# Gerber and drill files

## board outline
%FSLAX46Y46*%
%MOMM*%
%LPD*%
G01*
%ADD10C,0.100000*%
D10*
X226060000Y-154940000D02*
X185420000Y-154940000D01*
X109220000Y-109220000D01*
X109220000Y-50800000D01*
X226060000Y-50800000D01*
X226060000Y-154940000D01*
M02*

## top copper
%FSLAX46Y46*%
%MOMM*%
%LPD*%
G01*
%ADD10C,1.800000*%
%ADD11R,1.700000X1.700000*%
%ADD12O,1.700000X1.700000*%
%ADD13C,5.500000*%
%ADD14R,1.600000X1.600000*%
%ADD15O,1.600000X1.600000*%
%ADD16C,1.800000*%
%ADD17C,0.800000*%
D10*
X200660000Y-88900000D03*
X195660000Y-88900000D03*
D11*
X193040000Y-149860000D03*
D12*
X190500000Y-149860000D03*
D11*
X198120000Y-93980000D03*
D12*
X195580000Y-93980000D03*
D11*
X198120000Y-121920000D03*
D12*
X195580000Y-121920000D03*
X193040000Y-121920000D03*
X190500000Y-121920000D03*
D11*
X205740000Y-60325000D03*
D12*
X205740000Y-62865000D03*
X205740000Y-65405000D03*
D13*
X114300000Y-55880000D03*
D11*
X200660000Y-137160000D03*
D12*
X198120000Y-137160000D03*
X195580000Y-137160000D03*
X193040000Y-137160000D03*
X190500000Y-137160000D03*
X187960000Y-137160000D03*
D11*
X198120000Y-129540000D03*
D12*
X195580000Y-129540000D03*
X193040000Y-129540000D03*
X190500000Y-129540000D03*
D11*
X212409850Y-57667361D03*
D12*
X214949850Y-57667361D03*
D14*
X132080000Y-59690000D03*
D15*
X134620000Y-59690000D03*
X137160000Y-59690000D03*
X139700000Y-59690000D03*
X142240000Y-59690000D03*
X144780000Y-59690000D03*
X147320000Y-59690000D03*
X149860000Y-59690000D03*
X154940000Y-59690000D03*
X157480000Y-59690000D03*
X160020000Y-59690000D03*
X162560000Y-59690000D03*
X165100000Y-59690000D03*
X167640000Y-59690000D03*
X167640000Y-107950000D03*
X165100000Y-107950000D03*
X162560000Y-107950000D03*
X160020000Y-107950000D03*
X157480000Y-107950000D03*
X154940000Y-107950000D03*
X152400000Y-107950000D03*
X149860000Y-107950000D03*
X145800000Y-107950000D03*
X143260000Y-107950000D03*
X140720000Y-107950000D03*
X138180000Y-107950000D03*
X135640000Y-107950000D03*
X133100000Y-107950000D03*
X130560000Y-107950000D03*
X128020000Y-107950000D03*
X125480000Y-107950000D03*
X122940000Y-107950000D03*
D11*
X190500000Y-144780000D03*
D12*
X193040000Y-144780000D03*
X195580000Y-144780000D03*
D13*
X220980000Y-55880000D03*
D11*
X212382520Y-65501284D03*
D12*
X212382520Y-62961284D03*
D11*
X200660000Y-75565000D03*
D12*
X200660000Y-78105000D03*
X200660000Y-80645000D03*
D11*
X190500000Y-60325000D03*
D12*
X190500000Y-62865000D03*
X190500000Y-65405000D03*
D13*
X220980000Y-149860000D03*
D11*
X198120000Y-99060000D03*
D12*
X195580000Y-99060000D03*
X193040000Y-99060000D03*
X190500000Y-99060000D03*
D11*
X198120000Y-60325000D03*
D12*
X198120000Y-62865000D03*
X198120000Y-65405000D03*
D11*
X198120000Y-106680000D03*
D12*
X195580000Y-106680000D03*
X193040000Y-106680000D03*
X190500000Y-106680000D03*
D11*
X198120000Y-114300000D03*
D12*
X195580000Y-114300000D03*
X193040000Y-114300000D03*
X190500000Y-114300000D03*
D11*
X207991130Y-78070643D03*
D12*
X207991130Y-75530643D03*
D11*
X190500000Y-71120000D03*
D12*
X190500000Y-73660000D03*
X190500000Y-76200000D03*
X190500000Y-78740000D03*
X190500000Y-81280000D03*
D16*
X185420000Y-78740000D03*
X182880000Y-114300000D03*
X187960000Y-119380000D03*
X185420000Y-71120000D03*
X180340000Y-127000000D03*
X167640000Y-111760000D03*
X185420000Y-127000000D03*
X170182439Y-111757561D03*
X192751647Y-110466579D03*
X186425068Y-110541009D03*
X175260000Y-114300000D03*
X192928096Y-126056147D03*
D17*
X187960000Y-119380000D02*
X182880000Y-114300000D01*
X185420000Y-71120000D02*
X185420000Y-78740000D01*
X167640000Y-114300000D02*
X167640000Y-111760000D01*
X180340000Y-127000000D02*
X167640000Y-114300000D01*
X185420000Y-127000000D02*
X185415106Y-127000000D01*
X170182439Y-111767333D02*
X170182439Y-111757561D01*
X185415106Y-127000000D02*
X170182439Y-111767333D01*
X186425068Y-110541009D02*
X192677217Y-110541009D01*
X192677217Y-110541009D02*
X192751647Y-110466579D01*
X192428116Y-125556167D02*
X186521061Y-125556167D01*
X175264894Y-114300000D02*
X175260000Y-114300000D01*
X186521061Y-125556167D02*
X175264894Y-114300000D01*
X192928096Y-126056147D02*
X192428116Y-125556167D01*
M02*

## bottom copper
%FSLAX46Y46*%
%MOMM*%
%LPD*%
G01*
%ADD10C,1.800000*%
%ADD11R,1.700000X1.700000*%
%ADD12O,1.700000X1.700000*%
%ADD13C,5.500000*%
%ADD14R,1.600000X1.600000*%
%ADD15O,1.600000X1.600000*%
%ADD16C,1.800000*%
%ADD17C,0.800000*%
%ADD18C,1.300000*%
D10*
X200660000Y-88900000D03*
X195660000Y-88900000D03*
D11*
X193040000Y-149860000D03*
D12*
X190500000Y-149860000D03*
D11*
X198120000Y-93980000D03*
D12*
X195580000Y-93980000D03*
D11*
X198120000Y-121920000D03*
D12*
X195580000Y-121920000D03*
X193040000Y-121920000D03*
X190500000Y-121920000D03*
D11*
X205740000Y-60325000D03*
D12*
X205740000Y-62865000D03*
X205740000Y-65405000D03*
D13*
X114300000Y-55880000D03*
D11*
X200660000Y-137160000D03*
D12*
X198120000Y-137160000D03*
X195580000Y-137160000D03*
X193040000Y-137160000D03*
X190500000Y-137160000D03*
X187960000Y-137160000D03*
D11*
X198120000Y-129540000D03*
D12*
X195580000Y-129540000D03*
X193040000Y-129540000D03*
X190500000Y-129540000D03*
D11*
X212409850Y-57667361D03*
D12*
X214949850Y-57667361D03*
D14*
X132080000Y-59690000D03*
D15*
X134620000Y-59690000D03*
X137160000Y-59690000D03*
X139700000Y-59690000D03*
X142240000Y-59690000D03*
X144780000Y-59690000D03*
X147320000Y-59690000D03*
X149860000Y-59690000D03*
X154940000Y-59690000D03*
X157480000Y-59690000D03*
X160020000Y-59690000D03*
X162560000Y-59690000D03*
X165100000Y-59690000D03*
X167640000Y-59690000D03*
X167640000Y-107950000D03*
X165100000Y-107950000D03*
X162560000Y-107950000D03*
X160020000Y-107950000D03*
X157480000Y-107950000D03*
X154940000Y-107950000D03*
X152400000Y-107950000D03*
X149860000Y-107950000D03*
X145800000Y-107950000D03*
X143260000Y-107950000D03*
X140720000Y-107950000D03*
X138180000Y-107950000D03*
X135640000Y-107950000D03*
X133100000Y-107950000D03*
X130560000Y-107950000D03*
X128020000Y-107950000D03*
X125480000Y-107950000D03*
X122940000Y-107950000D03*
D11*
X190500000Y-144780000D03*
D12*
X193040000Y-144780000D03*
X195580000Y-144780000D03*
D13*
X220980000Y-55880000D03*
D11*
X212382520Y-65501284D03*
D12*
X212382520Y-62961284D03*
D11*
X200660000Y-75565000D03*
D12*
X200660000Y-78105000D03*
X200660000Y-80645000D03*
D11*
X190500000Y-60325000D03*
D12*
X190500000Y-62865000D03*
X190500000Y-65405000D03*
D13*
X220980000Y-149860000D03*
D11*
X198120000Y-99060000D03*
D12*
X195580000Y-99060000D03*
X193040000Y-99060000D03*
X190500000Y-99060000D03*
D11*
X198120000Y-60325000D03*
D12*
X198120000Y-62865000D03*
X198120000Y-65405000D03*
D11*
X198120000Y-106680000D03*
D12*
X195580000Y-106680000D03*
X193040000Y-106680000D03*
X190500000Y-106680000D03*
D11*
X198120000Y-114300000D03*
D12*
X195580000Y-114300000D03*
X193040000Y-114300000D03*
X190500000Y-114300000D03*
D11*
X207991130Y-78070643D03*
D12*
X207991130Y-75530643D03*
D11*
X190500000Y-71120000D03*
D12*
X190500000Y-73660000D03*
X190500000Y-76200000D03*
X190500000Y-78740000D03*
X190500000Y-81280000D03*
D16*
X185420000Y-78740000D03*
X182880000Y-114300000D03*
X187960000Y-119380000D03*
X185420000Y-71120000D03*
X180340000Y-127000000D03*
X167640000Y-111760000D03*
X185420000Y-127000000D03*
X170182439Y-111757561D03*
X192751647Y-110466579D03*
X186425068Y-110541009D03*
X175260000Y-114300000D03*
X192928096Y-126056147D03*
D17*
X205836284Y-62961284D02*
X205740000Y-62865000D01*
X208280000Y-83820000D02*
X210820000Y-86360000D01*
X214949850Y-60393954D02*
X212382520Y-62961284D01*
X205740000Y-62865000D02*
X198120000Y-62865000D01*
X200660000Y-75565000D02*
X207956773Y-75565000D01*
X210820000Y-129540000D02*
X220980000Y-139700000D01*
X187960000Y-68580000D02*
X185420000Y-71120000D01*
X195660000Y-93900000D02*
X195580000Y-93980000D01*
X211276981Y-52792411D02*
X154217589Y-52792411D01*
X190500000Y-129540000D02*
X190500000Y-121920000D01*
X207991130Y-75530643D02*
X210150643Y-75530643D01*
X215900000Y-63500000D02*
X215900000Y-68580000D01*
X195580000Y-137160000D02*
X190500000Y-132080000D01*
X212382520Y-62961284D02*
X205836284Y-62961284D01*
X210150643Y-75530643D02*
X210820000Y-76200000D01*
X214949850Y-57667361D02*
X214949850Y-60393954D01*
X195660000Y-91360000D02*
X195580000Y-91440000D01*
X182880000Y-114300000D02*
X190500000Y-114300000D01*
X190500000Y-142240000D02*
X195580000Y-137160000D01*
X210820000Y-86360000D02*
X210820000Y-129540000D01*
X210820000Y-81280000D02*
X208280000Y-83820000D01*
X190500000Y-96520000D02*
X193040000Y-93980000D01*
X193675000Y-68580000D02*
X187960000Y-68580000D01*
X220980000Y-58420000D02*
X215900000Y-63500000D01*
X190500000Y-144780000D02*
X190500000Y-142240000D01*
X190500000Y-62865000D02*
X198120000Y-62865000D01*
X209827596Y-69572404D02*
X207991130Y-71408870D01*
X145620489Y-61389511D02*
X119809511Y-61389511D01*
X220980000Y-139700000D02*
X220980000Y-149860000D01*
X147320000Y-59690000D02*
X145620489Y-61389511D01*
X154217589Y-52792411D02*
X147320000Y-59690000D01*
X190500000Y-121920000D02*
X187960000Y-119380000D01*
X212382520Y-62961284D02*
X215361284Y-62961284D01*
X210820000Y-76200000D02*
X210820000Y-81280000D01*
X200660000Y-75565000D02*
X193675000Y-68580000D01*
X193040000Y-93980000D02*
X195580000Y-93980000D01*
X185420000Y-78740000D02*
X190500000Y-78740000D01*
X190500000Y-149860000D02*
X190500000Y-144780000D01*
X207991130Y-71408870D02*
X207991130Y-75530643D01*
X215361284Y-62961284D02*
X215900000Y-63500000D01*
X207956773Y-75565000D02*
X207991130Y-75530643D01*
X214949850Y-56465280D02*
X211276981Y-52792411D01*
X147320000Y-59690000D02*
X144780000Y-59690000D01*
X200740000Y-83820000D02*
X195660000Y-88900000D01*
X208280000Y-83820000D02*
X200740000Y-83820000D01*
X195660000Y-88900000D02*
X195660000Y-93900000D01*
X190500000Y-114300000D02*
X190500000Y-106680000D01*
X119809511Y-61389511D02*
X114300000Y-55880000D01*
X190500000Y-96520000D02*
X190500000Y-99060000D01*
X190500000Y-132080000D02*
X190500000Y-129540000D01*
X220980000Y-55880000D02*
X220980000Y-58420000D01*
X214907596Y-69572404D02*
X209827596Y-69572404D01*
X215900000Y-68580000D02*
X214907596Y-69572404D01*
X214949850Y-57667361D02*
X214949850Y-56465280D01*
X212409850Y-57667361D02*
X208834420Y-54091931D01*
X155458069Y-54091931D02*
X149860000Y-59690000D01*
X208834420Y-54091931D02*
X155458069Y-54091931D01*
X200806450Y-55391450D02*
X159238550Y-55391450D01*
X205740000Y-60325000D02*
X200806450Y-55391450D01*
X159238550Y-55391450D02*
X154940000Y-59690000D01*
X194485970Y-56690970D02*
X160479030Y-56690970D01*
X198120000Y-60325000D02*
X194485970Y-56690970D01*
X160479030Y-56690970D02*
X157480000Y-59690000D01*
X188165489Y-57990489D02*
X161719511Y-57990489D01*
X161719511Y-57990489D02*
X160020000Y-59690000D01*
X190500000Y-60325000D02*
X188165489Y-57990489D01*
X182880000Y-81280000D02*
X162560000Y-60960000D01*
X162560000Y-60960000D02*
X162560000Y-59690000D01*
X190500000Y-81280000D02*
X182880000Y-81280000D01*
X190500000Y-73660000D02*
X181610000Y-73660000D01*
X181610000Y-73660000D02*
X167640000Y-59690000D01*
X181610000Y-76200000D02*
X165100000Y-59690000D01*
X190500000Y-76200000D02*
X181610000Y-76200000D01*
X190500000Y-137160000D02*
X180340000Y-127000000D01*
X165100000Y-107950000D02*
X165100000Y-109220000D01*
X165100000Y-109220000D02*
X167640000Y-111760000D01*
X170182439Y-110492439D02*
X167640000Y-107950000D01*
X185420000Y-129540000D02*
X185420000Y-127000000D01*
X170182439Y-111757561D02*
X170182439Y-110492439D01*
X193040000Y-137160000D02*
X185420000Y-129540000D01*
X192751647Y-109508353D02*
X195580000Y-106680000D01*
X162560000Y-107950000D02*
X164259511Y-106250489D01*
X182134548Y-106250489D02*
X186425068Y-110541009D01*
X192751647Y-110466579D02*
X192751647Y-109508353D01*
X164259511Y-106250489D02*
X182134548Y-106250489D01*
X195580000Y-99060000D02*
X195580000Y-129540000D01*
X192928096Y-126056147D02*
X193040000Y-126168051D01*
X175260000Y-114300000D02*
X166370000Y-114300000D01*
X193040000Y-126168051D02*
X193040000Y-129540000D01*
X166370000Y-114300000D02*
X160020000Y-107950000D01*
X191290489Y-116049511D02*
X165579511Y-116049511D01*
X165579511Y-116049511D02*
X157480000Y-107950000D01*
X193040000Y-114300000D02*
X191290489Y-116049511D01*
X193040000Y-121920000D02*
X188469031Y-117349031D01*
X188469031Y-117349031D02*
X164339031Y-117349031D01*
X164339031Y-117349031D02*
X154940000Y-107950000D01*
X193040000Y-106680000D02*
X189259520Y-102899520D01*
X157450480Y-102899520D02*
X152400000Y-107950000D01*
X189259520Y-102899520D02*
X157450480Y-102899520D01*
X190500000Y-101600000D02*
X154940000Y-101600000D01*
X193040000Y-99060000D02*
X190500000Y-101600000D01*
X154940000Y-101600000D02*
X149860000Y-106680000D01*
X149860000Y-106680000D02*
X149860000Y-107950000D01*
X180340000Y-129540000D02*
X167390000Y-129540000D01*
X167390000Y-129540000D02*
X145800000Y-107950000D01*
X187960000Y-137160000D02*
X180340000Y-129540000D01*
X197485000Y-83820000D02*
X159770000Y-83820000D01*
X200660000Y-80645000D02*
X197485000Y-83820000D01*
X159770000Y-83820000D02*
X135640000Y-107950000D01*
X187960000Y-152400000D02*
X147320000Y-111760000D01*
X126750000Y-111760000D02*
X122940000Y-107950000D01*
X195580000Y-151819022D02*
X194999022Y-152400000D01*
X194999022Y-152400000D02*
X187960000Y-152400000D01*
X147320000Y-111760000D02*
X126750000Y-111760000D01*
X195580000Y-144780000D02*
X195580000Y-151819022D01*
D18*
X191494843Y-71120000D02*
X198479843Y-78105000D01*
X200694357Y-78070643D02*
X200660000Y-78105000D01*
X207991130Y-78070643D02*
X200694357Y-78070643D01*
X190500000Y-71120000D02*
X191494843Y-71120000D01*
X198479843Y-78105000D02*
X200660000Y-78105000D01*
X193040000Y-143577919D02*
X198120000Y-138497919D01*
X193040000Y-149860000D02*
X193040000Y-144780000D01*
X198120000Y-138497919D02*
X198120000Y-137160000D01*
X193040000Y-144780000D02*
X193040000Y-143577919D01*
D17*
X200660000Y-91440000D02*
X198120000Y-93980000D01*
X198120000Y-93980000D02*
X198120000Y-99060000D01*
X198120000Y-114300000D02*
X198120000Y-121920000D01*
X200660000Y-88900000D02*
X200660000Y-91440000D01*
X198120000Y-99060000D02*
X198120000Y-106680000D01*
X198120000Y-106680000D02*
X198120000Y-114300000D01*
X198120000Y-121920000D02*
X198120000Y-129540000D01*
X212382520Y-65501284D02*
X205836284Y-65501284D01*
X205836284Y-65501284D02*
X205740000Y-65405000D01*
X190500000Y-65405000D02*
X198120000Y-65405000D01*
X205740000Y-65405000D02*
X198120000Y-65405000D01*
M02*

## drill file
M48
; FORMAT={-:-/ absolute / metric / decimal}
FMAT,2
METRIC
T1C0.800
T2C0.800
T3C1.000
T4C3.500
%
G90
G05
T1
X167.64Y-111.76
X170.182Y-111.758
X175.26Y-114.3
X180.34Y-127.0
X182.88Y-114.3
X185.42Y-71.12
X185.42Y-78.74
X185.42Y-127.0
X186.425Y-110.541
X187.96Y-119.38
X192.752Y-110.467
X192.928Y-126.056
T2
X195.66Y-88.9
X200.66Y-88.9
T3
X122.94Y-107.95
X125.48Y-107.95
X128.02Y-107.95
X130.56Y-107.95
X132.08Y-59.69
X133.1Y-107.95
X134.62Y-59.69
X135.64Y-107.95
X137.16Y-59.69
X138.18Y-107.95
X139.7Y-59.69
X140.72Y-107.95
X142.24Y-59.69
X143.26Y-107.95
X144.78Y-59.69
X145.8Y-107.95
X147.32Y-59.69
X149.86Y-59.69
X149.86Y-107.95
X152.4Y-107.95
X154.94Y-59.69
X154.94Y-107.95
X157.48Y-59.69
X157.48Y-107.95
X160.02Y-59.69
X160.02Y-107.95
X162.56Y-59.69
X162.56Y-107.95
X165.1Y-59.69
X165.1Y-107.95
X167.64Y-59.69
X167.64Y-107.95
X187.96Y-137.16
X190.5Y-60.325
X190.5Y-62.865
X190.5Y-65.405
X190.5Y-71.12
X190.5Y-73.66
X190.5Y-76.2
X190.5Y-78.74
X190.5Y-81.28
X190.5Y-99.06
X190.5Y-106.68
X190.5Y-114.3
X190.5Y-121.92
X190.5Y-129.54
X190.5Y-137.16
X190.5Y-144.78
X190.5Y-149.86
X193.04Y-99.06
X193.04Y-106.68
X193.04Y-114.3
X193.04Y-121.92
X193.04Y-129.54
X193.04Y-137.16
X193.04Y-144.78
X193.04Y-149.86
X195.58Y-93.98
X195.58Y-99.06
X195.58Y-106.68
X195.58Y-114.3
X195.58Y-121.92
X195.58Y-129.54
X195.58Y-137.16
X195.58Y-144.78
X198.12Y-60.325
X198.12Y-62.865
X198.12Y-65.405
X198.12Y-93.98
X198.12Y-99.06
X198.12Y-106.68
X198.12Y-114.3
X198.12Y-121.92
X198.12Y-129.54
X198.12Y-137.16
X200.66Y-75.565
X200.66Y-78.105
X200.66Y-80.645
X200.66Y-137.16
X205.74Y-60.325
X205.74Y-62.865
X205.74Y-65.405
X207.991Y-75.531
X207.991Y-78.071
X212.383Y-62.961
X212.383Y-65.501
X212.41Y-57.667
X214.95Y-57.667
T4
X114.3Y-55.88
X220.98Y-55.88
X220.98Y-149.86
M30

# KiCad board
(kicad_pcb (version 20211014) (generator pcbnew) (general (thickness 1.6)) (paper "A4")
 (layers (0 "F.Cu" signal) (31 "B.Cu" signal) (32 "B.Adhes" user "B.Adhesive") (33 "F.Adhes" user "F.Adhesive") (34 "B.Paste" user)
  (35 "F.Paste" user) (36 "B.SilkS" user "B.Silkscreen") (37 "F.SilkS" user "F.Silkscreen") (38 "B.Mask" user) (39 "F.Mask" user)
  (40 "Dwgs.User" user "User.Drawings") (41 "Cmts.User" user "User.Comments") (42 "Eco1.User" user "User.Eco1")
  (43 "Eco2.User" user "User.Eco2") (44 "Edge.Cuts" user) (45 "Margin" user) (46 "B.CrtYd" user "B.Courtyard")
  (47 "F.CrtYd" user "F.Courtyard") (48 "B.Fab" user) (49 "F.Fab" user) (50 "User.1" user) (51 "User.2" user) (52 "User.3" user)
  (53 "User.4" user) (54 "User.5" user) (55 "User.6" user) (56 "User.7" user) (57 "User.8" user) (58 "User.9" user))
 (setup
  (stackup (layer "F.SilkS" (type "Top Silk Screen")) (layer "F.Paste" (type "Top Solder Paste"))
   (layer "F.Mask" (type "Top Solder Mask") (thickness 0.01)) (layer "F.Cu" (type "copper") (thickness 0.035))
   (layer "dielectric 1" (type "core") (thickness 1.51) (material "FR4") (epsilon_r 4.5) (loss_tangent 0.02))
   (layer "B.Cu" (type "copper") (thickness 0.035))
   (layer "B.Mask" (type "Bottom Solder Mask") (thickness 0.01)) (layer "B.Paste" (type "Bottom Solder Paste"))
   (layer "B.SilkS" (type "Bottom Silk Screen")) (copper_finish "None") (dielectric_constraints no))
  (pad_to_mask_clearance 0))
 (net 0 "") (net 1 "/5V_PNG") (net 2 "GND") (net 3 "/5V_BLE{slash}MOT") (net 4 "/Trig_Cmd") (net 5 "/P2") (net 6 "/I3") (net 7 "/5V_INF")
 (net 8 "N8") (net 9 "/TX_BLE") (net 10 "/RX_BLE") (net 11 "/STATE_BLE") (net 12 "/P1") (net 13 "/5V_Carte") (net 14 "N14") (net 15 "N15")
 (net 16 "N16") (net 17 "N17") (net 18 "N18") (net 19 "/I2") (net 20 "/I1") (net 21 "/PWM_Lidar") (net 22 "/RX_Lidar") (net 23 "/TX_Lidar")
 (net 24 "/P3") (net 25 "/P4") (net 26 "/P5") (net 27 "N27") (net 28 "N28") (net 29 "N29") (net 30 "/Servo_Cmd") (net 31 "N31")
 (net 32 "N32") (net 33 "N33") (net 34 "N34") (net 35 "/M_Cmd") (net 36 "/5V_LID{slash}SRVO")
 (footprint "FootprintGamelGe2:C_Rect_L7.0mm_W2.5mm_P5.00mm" (layer "F.Cu") (at 200.66 88.9 180)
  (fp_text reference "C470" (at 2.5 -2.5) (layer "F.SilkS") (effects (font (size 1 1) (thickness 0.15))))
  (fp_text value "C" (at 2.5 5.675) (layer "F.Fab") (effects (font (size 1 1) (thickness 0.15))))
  (pad "1" thru_hole circle locked (at 0 0 180) (size 1.8 1.8) (drill 0.8) (layers *.Cu *.Mask) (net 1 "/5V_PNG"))
  (pad "2" thru_hole circle locked (at 5 0 180) (size 1.8 1.8) (drill 0.8) (layers *.Cu *.Mask) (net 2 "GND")))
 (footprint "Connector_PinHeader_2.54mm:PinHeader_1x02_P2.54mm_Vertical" (layer "F.Cu") (at 193.04 149.86 -90)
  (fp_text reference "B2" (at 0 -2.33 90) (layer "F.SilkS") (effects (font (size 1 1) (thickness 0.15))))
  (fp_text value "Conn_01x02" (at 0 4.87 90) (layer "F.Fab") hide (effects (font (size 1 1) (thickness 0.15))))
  (pad "1" thru_hole rect (at 0 0 270) (size 1.7 1.7) (drill 1) (layers *.Cu *.Mask) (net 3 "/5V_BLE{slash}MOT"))
  (pad "2" thru_hole oval (at 0 2.54 270) (size 1.7 1.7) (drill 1) (layers *.Cu *.Mask) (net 2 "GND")))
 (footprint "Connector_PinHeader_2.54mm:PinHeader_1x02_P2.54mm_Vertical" (layer "F.Cu") (at 198.12 93.98 -90)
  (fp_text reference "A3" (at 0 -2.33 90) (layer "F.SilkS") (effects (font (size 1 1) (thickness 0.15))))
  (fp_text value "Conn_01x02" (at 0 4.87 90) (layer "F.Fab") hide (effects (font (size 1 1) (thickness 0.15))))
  (pad "1" thru_hole rect (at 0 0 270) (size 1.7 1.7) (drill 1) (layers *.Cu *.Mask) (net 1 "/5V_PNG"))
  (pad "2" thru_hole oval (at 0 2.54 270) (size 1.7 1.7) (drill 1) (layers *.Cu *.Mask) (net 2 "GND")))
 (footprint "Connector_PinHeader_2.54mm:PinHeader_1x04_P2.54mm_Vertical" (layer "F.Cu") (at 198.12 121.92 -90)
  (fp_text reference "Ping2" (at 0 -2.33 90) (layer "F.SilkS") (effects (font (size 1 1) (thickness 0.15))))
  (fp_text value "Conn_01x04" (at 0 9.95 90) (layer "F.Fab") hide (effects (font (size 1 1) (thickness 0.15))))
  (pad "1" thru_hole rect (at 0 0 270) (size 1.7 1.7) (drill 1) (layers *.Cu *.Mask) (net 1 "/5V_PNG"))
  (pad "2" thru_hole oval (at 0 2.54 270) (size 1.7 1.7) (drill 1) (layers *.Cu *.Mask) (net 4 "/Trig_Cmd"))
  (pad "3" thru_hole oval (at 0 5.08 270) (size 1.7 1.7) (drill 1) (layers *.Cu *.Mask) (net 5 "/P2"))
  (pad "4" thru_hole oval (at 0 7.62 270) (size 1.7 1.7) (drill 1) (layers *.Cu *.Mask) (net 2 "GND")))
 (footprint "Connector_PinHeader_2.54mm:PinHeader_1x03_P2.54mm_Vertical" (layer "F.Cu") (at 205.74 60.325)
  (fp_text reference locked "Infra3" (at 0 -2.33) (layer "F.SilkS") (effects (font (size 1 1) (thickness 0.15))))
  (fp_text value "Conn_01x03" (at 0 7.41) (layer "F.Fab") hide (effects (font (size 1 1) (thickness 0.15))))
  (pad "1" thru_hole rect (at 0 0) (size 1.7 1.7) (drill 1) (layers *.Cu *.Mask) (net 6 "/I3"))
  (pad "2" thru_hole oval (at 0 2.54) (size 1.7 1.7) (drill 1) (layers *.Cu *.Mask) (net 2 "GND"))
  (pad "3" thru_hole oval (at 0 5.08) (size 1.7 1.7) (drill 1) (layers *.Cu *.Mask) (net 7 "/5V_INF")))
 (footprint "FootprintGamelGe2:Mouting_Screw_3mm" (layer "F.Cu") (at 114.3 55.88)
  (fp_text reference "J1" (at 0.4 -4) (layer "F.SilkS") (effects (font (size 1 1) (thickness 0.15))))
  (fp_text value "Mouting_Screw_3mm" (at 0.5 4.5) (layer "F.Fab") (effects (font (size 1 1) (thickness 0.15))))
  (pad "1" thru_hole circle locked (at 0 0) (size 5.5 5.5) (drill 3.5) (layers *.Cu *.Mask) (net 2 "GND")))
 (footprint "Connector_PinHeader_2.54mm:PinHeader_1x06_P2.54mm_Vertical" (layer "F.Cu") (at 200.66 137.16 -90)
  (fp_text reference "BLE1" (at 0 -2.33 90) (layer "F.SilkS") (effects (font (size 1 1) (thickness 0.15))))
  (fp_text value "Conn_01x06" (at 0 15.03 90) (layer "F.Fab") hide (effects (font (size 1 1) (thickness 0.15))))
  (pad "1" thru_hole rect (at 0 0 270) (size 1.7 1.7) (drill 1) (layers *.Cu *.Mask) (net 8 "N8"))
  (pad "2" thru_hole oval (at 0 2.54 270) (size 1.7 1.7) (drill 1) (layers *.Cu *.Mask) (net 3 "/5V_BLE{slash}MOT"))
  (pad "3" thru_hole oval (at 0 5.08 270) (size 1.7 1.7) (drill 1) (layers *.Cu *.Mask) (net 2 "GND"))
  (pad "4" thru_hole oval (at 0 7.62 270) (size 1.7 1.7) (drill 1) (layers *.Cu *.Mask) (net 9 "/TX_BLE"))
  (pad "5" thru_hole oval (at 0 10.16 270) (size 1.7 1.7) (drill 1) (layers *.Cu *.Mask) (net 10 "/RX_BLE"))
  (pad "6" thru_hole oval (at 0 12.7 270) (size 1.7 1.7) (drill 1) (layers *.Cu *.Mask) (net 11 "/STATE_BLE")))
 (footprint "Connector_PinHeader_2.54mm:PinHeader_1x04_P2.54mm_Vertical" (layer "F.Cu") (at 198.12 129.54 -90)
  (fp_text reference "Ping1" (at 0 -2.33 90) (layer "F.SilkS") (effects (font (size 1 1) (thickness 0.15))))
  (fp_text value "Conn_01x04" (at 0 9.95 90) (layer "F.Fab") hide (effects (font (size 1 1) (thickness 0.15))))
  (pad "1" thru_hole rect (at 0 0 270) (size 1.7 1.7) (drill 1) (layers *.Cu *.Mask) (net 1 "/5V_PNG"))
  (pad "2" thru_hole oval (at 0 2.54 270) (size 1.7 1.7) (drill 1) (layers *.Cu *.Mask) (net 4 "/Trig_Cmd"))
  (pad "3" thru_hole oval (at 0 5.08 270) (size 1.7 1.7) (drill 1) (layers *.Cu *.Mask) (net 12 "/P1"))
  (pad "4" thru_hole oval (at 0 7.62 270) (size 1.7 1.7) (drill 1) (layers *.Cu *.Mask) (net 2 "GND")))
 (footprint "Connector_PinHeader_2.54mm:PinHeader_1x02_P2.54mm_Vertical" (layer "F.Cu") (at 212.40985 57.667361 90)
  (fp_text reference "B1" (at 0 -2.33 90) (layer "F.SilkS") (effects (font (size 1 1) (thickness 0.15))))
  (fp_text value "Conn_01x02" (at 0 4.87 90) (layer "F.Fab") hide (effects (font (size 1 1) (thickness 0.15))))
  (pad "1" thru_hole rect (at 0 0 90) (size 1.7 1.7) (drill 1) (layers *.Cu *.Mask) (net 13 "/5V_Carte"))
  (pad "2" thru_hole oval (at 0 2.54 90) (size 1.7 1.7) (drill 1) (layers *.Cu *.Mask) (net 2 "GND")))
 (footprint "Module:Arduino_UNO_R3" (layer "F.Cu") (at 132.08 59.69)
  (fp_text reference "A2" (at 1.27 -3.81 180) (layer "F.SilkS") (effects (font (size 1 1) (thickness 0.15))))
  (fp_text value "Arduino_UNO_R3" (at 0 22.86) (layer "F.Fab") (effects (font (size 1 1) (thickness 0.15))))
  (pad "1" thru_hole rect (at 0 0 90) (size 1.6 1.6) (drill 1) (layers *.Cu *.Mask) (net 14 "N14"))
  (pad "2" thru_hole oval (at 2.54 0 90) (size 1.6 1.6) (drill 1) (layers *.Cu *.Mask) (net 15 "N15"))
  (pad "3" thru_hole oval (at 5.08 0 90) (size 1.6 1.6) (drill 1) (layers *.Cu *.Mask) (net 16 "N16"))
  (pad "4" thru_hole oval (at 7.62 0 90) (size 1.6 1.6) (drill 1) (layers *.Cu *.Mask) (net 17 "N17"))
  (pad "5" thru_hole oval (at 10.16 0 90) (size 1.6 1.6) (drill 1) (layers *.Cu *.Mask) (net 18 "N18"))
  (pad "6" thru_hole oval (at 12.7 0 90) (size 1.6 1.6) (drill 1) (layers *.Cu *.Mask) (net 2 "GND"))
  (pad "7" thru_hole oval (at 15.24 0 90) (size 1.6 1.6) (drill 1) (layers *.Cu *.Mask) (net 2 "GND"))
  (pad "8" thru_hole oval (at 17.78 0 90) (size 1.6 1.6) (drill 1) (layers *.Cu *.Mask) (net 13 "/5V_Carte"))
  (pad "9" thru_hole oval (at 22.86 0 90) (size 1.6 1.6) (drill 1) (layers *.Cu *.Mask) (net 6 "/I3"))
  (pad "10" thru_hole oval (at 25.4 0 90) (size 1.6 1.6) (drill 1) (layers *.Cu *.Mask) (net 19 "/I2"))
  (pad "11" thru_hole oval (at 27.94 0 90) (size 1.6 1.6) (drill 1) (layers *.Cu *.Mask) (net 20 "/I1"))
  (pad "12" thru_hole oval (at 30.48 0 90) (size 1.6 1.6) (drill 1) (layers *.Cu *.Mask) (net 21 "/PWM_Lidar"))
  (pad "13" thru_hole oval (at 33.02 0 90) (size 1.6 1.6) (drill 1) (layers *.Cu *.Mask) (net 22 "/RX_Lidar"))
  (pad "14" thru_hole oval (at 35.56 0 90) (size 1.6 1.6) (drill 1) (layers *.Cu *.Mask) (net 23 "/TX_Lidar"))
  (pad "15" thru_hole oval (at 35.56 48.26 90) (size 1.6 1.6) (drill 1) (layers *.Cu *.Mask) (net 9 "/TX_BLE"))
  (pad "16" thru_hole oval (at 33.02 48.26 90) (size 1.6 1.6) (drill 1) (layers *.Cu *.Mask) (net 10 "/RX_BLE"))
  (pad "17" thru_hole oval (at 30.48 48.26 90) (size 1.6 1.6) (drill 1) (layers *.Cu *.Mask) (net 4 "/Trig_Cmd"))
  (pad "18" thru_hole oval (at 27.94 48.26 90) (size 1.6 1.6) (drill 1) (layers *.Cu *.Mask) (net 12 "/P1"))
  (pad "19" thru_hole oval (at 25.4 48.26 90) (size 1.6 1.6) (drill 1) (layers *.Cu *.Mask) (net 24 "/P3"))
  (pad "20" thru_hole oval (at 22.86 48.26 90) (size 1.6 1.6) (drill 1) (layers *.Cu *.Mask) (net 5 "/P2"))
  (pad "21" thru_hole oval (at 20.32 48.26 90) (size 1.6 1.6) (drill 1) (layers *.Cu *.Mask) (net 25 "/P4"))
  (pad "22" thru_hole oval (at 17.78 48.26 90) (size 1.6 1.6) (drill 1) (layers *.Cu *.Mask) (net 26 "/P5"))
  (pad "23" thru_hole oval (at 13.72 48.26 90) (size 1.6 1.6) (drill 1) (layers *.Cu *.Mask) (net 11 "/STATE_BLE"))
  (pad "24" thru_hole oval (at 11.18 48.26 90) (size 1.6 1.6) (drill 1) (layers *.Cu *.Mask) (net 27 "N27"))
  (pad "25" thru_hole oval (at 8.64 48.26 90) (size 1.6 1.6) (drill 1) (layers *.Cu *.Mask) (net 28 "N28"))
  (pad "26" thru_hole oval (at 6.1 48.26 90) (size 1.6 1.6) (drill 1) (layers *.Cu *.Mask) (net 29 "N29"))
  (pad "27" thru_hole oval (at 3.56 48.26 90) (size 1.6 1.6) (drill 1) (layers *.Cu *.Mask) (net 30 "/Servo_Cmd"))
  (pad "28" thru_hole oval (at 1.02 48.26 90) (size 1.6 1.6) (drill 1) (layers *.Cu *.Mask) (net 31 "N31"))
  (pad "29" thru_hole oval (at -1.52 48.26 90) (size 1.6 1.6) (drill 1) (layers *.Cu *.Mask) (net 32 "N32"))
  (pad "30" thru_hole oval (at -4.06 48.26 90) (size 1.6 1.6) (drill 1) (layers *.Cu *.Mask) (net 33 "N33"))
  (pad "31" thru_hole oval (at -6.6 48.26 90) (size 1.6 1.6) (drill 1) (layers *.Cu *.Mask) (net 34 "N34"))
  (pad "32" thru_hole oval (at -9.14 48.26 90) (size 1.6 1.6) (drill 1) (layers *.Cu *.Mask) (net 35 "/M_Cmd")))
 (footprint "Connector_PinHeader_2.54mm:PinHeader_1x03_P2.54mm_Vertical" (layer "F.Cu") (at 190.5 144.78 90)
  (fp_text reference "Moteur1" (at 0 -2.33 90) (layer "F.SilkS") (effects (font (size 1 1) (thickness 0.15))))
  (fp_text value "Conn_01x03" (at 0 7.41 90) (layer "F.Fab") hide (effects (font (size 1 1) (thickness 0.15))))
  (pad "1" thru_hole rect (at 0 0 90) (size 1.7 1.7) (drill 1) (layers *.Cu *.Mask) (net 2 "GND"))
  (pad "2" thru_hole oval (at 0 2.54 90) (size 1.7 1.7) (drill 1) (layers *.Cu *.Mask) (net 3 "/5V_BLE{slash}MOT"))
  (pad "3" thru_hole oval (at 0 5.08 90) (size 1.7 1.7) (drill 1) (layers *.Cu *.Mask) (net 35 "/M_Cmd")))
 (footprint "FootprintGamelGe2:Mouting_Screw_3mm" (layer "F.Cu") (at 220.98 55.88)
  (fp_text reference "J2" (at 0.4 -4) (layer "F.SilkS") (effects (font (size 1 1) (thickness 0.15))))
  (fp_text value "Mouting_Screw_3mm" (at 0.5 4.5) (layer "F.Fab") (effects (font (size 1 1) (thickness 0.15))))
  (pad "1" thru_hole circle locked (at 0 0) (size 5.5 5.5) (drill 3.5) (layers *.Cu *.Mask) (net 2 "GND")))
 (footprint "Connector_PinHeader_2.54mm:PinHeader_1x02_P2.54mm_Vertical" (layer "F.Cu") (at 212.38252 65.501284 180)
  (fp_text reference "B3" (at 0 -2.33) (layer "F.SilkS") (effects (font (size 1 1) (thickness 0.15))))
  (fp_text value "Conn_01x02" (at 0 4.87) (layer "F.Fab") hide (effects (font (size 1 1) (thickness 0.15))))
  (pad "1" thru_hole rect (at 0 0 180) (size 1.7 1.7) (drill 1) (layers *.Cu *.Mask) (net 7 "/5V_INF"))
  (pad "2" thru_hole oval (at 0 2.54 180) (size 1.7 1.7) (drill 1) (layers *.Cu *.Mask) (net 2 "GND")))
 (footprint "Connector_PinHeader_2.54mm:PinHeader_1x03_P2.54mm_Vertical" (layer "F.Cu") (at 200.66 75.565)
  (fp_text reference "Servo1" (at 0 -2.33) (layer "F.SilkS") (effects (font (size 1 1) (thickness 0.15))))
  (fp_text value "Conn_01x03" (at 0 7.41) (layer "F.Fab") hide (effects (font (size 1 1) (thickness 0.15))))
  (pad "1" thru_hole rect (at 0 0) (size 1.7 1.7) (drill 1) (layers *.Cu *.Mask) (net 2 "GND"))
  (pad "2" thru_hole oval (at 0 2.54) (size 1.7 1.7) (drill 1) (layers *.Cu *.Mask) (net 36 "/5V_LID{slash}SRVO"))
  (pad "3" thru_hole oval (at 0 5.08) (size 1.7 1.7) (drill 1) (layers *.Cu *.Mask) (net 30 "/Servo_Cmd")))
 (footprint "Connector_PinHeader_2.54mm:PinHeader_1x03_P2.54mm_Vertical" (layer "F.Cu") (at 190.5 60.325)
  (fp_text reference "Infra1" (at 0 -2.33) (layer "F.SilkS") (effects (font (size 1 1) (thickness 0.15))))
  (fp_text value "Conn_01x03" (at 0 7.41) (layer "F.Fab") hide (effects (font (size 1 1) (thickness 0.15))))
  (pad "1" thru_hole rect (at 0 0) (size 1.7 1.7) (drill 1) (layers *.Cu *.Mask) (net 20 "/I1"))
  (pad "2" thru_hole oval (at 0 2.54) (size 1.7 1.7) (drill 1) (layers *.Cu *.Mask) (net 2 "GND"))
  (pad "3" thru_hole oval (at 0 5.08) (size 1.7 1.7) (drill 1) (layers *.Cu *.Mask) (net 7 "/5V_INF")))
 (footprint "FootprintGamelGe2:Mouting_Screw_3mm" (layer "F.Cu") (at 220.98 149.86)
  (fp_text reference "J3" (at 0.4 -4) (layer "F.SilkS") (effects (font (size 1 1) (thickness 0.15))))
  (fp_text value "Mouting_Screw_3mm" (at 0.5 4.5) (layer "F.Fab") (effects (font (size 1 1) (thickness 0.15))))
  (pad "1" thru_hole circle locked (at 0 0) (size 5.5 5.5) (drill 3.5) (layers *.Cu *.Mask) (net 2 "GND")))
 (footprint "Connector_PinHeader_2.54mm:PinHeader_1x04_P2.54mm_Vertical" (layer "F.Cu") (at 198.12 99.06 -90)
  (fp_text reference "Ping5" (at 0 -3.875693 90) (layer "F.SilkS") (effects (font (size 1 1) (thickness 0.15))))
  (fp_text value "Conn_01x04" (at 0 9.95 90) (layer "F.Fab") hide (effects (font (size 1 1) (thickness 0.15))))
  (pad "1" thru_hole rect (at 0 0 270) (size 1.7 1.7) (drill 1) (layers *.Cu *.Mask) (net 1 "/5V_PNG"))
  (pad "2" thru_hole oval (at 0 2.54 270) (size 1.7 1.7) (drill 1) (layers *.Cu *.Mask) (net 4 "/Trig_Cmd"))
  (pad "3" thru_hole oval (at 0 5.08 270) (size 1.7 1.7) (drill 1) (layers *.Cu *.Mask) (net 26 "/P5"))
  (pad "4" thru_hole oval (at 0 7.62 270) (size 1.7 1.7) (drill 1) (layers *.Cu *.Mask) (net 2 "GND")))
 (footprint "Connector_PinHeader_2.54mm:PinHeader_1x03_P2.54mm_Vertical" (layer "F.Cu") (at 198.12 60.325)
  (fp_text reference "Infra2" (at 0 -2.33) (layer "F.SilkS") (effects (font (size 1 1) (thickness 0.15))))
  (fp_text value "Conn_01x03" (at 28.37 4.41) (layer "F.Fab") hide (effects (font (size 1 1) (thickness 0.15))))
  (pad "1" thru_hole rect (at 0 0) (size 1.7 1.7) (drill 1) (layers *.Cu *.Mask) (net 19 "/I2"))
  (pad "2" thru_hole oval (at 0 2.54) (size 1.7 1.7) (drill 1) (layers *.Cu *.Mask) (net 2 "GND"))
  (pad "3" thru_hole oval (at 0 5.08) (size 1.7 1.7) (drill 1) (layers *.Cu *.Mask) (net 7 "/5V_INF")))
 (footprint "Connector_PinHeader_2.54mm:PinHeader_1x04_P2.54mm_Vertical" (layer "F.Cu") (at 198.12 106.68 -90)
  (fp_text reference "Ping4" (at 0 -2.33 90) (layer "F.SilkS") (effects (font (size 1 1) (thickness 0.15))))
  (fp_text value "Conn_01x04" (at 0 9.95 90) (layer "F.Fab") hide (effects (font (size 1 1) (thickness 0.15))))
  (pad "1" thru_hole rect (at 0 0 270) (size 1.7 1.7) (drill 1) (layers *.Cu *.Mask) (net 1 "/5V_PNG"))
  (pad "2" thru_hole oval (at 0 2.54 270) (size 1.7 1.7) (drill 1) (layers *.Cu *.Mask) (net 4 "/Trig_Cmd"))
  (pad "3" thru_hole oval (at 0 5.08 270) (size 1.7 1.7) (drill 1) (layers *.Cu *.Mask) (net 25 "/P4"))
  (pad "4" thru_hole oval (at 0 7.62 270) (size 1.7 1.7) (drill 1) (layers *.Cu *.Mask) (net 2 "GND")))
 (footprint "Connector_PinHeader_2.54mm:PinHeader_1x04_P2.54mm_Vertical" (layer "F.Cu") (at 198.12 114.3 -90)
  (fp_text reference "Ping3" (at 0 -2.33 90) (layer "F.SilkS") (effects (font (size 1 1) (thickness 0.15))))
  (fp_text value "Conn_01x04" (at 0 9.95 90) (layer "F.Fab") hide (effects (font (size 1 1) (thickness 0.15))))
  (pad "1" thru_hole rect (at 0 0 270) (size 1.7 1.7) (drill 1) (layers *.Cu *.Mask) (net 1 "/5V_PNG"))
  (pad "2" thru_hole oval (at 0 2.54 270) (size 1.7 1.7) (drill 1) (layers *.Cu *.Mask) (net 4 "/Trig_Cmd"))
  (pad "3" thru_hole oval (at 0 5.08 270) (size 1.7 1.7) (drill 1) (layers *.Cu *.Mask) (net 24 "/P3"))
  (pad "4" thru_hole oval (at 0 7.62 270) (size 1.7 1.7) (drill 1) (layers *.Cu *.Mask) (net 2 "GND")))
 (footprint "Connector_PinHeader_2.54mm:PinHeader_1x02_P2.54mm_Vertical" (layer "F.Cu") (at 207.99113 78.070643 180)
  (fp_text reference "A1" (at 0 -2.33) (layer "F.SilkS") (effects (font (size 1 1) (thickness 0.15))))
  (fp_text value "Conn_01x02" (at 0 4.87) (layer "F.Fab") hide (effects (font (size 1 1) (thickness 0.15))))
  (pad "1" thru_hole rect (at 0 0 180) (size 1.7 1.7) (drill 1) (layers *.Cu *.Mask) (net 36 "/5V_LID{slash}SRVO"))
  (pad "2" thru_hole oval (at 0 2.54 180) (size 1.7 1.7) (drill 1) (layers *.Cu *.Mask) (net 2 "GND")))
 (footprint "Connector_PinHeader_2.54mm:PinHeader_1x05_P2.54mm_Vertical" (layer "F.Cu") (at 190.5 71.12)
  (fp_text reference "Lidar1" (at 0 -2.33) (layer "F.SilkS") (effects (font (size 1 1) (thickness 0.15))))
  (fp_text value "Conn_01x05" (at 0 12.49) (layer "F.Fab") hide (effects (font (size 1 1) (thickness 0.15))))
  (pad "1" thru_hole rect (at 0 0) (size 1.7 1.7) (drill 1) (layers *.Cu *.Mask) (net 36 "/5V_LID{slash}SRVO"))
  (pad "2" thru_hole oval (at 0 2.54) (size 1.7 1.7) (drill 1) (layers *.Cu *.Mask) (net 23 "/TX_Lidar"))
  (pad "3" thru_hole oval (at 0 5.08) (size 1.7 1.7) (drill 1) (layers *.Cu *.Mask) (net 22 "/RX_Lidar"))
  (pad "4" thru_hole oval (at 0 7.62) (size 1.7 1.7) (drill 1) (layers *.Cu *.Mask) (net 2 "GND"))
  (pad "5" thru_hole oval (at 0 10.16) (size 1.7 1.7) (drill 1) (layers *.Cu *.Mask) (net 21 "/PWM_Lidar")))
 (gr_poly
  (pts (xy 226.06 154.94) (xy 185.42 154.94) (xy 109.22 109.22) (xy 109.22 50.8) (xy 226.06 50.8)) (layer "Edge.Cuts") (width 0.1)
  (fill none))
 (segment (start 187.96 119.38) (end 182.88 114.3) (width 0.8) (layer "F.Cu") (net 2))
 (segment (start 185.42 71.12) (end 185.42 78.74) (width 0.8) (layer "F.Cu") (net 2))
 (via (at 185.42 78.74) (size 1.8) (drill 0.8) (layers "F.Cu" "B.Cu") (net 2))
 (via (at 182.88 114.3) (size 1.8) (drill 0.8) (layers "F.Cu" "B.Cu") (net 2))
 (via (at 187.96 119.38) (size 1.8) (drill 0.8) (layers "F.Cu" "B.Cu") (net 2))
 (via (at 185.42 71.12) (size 1.8) (drill 0.8) (layers "F.Cu" "B.Cu") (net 2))
 (segment (start 205.836284 62.961284) (end 205.74 62.865) (width 0.8) (layer "B.Cu") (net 2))
 (segment (start 208.28 83.82) (end 210.82 86.36) (width 0.8) (layer "B.Cu") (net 2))
 (segment (start 214.94985 60.393954) (end 212.38252 62.961284) (width 0.8) (layer "B.Cu") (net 2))
 (segment (start 205.74 62.865) (end 198.12 62.865) (width 0.8) (layer "B.Cu") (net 2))
 (segment (start 200.66 75.565) (end 207.956773 75.565) (width 0.8) (layer "B.Cu") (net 2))
 (segment (start 210.82 129.54) (end 220.98 139.7) (width 0.8) (layer "B.Cu") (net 2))
 (segment (start 187.96 68.58) (end 185.42 71.12) (width 0.8) (layer "B.Cu") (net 2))
 (segment (start 195.66 93.9) (end 195.58 93.98) (width 0.8) (layer "B.Cu") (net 2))
 (segment (start 211.276981 52.792411) (end 154.217589 52.792411) (width 0.8) (layer "B.Cu") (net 2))
 (segment (start 190.5 129.54) (end 190.5 121.92) (width 0.8) (layer "B.Cu") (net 2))
 (segment (start 207.99113 75.530643) (end 210.150643 75.530643) (width 0.8) (layer "B.Cu") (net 2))
 (segment (start 215.9 63.5) (end 215.9 68.58) (width 0.8) (layer "B.Cu") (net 2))
 (segment (start 195.58 137.16) (end 190.5 132.08) (width 0.8) (layer "B.Cu") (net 2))
 (segment (start 212.38252 62.961284) (end 205.836284 62.961284) (width 0.8) (layer "B.Cu") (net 2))
 (segment (start 210.150643 75.530643) (end 210.82 76.2) (width 0.8) (layer "B.Cu") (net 2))
 (segment (start 214.94985 57.667361) (end 214.94985 60.393954) (width 0.8) (layer "B.Cu") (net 2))
 (segment (start 195.66 91.36) (end 195.58 91.44) (width 0.8) (layer "B.Cu") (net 2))
 (segment (start 182.88 114.3) (end 190.5 114.3) (width 0.8) (layer "B.Cu") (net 2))
 (segment (start 190.5 142.24) (end 195.58 137.16) (width 0.8) (layer "B.Cu") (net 2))
 (segment (start 210.82 86.36) (end 210.82 129.54) (width 0.8) (layer "B.Cu") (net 2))
 (segment (start 210.82 81.28) (end 208.28 83.82) (width 0.8) (layer "B.Cu") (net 2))
 (segment (start 190.5 96.52) (end 193.04 93.98) (width 0.8) (layer "B.Cu") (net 2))
 (segment (start 193.675 68.58) (end 187.96 68.58) (width 0.8) (layer "B.Cu") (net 2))
 (segment (start 220.98 58.42) (end 215.9 63.5) (width 0.8) (layer "B.Cu") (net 2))
 (segment (start 190.5 144.78) (end 190.5 142.24) (width 0.8) (layer "B.Cu") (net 2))
 (segment (start 190.5 62.865) (end 198.12 62.865) (width 0.8) (layer "B.Cu") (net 2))
 (segment (start 209.827596 69.572404) (end 207.99113 71.40887) (width 0.8) (layer "B.Cu") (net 2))
 (segment (start 145.620489 61.389511) (end 119.809511 61.389511) (width 0.8) (layer "B.Cu") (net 2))
 (segment (start 220.98 139.7) (end 220.98 149.86) (width 0.8) (layer "B.Cu") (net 2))
 (segment (start 147.32 59.69) (end 145.620489 61.389511) (width 0.8) (layer "B.Cu") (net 2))
 (segment (start 154.217589 52.792411) (end 147.32 59.69) (width 0.8) (layer "B.Cu") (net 2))
 (segment (start 190.5 121.92) (end 187.96 119.38) (width 0.8) (layer "B.Cu") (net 2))
 (segment (start 212.38252 62.961284) (end 215.361284 62.961284) (width 0.8) (layer "B.Cu") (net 2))
 (segment (start 210.82 76.2) (end 210.82 81.28) (width 0.8) (layer "B.Cu") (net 2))
 (segment (start 200.66 75.565) (end 193.675 68.58) (width 0.8) (layer "B.Cu") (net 2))
 (segment (start 193.04 93.98) (end 195.58 93.98) (width 0.8) (layer "B.Cu") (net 2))
 (segment (start 185.42 78.74) (end 190.5 78.74) (width 0.8) (layer "B.Cu") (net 2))
 (segment (start 190.5 149.86) (end 190.5 144.78) (width 0.8) (layer "B.Cu") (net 2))
 (segment (start 207.99113 71.40887) (end 207.99113 75.530643) (width 0.8) (layer "B.Cu") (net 2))
 (segment (start 215.361284 62.961284) (end 215.9 63.5) (width 0.8) (layer "B.Cu") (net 2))
 (segment (start 207.956773 75.565) (end 207.99113 75.530643) (width 0.8) (layer "B.Cu") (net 2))
 (segment (start 214.94985 56.46528) (end 211.276981 52.792411) (width 0.8) (layer "B.Cu") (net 2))
 (segment (start 147.32 59.69) (end 144.78 59.69) (width 0.8) (layer "B.Cu") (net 2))
 (segment (start 200.74 83.82) (end 195.66 88.9) (width 0.8) (layer "B.Cu") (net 2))
 (segment (start 208.28 83.82) (end 200.74 83.82) (width 0.8) (layer "B.Cu") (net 2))
 (segment (start 195.66 88.9) (end 195.66 93.9) (width 0.8) (layer "B.Cu") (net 2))
 (segment (start 190.5 114.3) (end 190.5 106.68) (width 0.8) (layer "B.Cu") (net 2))
 (segment (start 119.809511 61.389511) (end 114.3 55.88) (width 0.8) (layer "B.Cu") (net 2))
 (segment (start 190.5 96.52) (end 190.5 99.06) (width 0.8) (layer "B.Cu") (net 2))
 (segment (start 190.5 132.08) (end 190.5 129.54) (width 0.8) (layer "B.Cu") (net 2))
 (segment (start 220.98 55.88) (end 220.98 58.42) (width 0.8) (layer "B.Cu") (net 2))
 (segment (start 214.907596 69.572404) (end 209.827596 69.572404) (width 0.8) (layer "B.Cu") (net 2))
 (segment (start 215.9 68.58) (end 214.907596 69.572404) (width 0.8) (layer "B.Cu") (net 2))
 (segment (start 214.94985 57.667361) (end 214.94985 56.46528) (width 0.8) (layer "B.Cu") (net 2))
 (segment (start 212.40985 57.667361) (end 208.83442 54.091931) (width 0.8) (layer "B.Cu") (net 13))
 (segment (start 155.458069 54.091931) (end 149.86 59.69) (width 0.8) (layer "B.Cu") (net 13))
 (segment (start 208.83442 54.091931) (end 155.458069 54.091931) (width 0.8) (layer "B.Cu") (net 13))
 (segment (start 200.80645 55.39145) (end 159.23855 55.39145) (width 0.8) (layer "B.Cu") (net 6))
 (segment (start 205.74 60.325) (end 200.80645 55.39145) (width 0.8) (layer "B.Cu") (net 6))
 (segment (start 159.23855 55.39145) (end 154.94 59.69) (width 0.8) (layer "B.Cu") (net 6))
 (segment (start 194.48597 56.69097) (end 160.47903 56.69097) (width 0.8) (layer "B.Cu") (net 19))
 (segment (start 198.12 60.325) (end 194.48597 56.69097) (width 0.8) (layer "B.Cu") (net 19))
 (segment (start 160.47903 56.69097) (end 157.48 59.69) (width 0.8) (layer "B.Cu") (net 19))
 (segment (start 188.165489 57.990489) (end 161.719511 57.990489) (width 0.8) (layer "B.Cu") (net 20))
 (segment (start 161.719511 57.990489) (end 160.02 59.69) (width 0.8) (layer "B.Cu") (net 20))
 (segment (start 190.5 60.325) (end 188.165489 57.990489) (width 0.8) (layer "B.Cu") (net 20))
 (segment (start 182.88 81.28) (end 162.56 60.96) (width 0.8) (layer "B.Cu") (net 21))
 (segment (start 162.56 60.96) (end 162.56 59.69) (width 0.8) (layer "B.Cu") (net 21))
 (segment (start 190.5 81.28) (end 182.88 81.28) (width 0.8) (layer "B.Cu") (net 21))
 (segment (start 190.5 73.66) (end 181.61 73.66) (width 0.8) (layer "B.Cu") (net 23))
 (segment (start 181.61 73.66) (end 167.64 59.69) (width 0.8) (layer "B.Cu") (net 23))
 (segment (start 181.61 76.2) (end 165.1 59.69) (width 0.8) (layer "B.Cu") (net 22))
 (segment (start 190.5 76.2) (end 181.61 76.2) (width 0.8) (layer "B.Cu") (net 22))
 (segment (start 167.64 114.3) (end 167.64 111.76) (width 0.8) (layer "F.Cu") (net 10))
 (segment (start 180.34 127) (end 167.64 114.3) (width 0.8) (layer "F.Cu") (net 10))
 (via (at 180.34 127) (size 1.8) (drill 0.8) (layers "F.Cu" "B.Cu") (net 10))
 (via (at 167.64 111.76) (size 1.8) (drill 0.8) (layers "F.Cu" "B.Cu") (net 10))
 (segment (start 190.5 137.16) (end 180.34 127) (width 0.8) (layer "B.Cu") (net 10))
 (segment (start 165.1 107.95) (end 165.1 109.22) (width 0.8) (layer "B.Cu") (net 10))
 (segment (start 165.1 109.22) (end 167.64 111.76) (width 0.8) (layer "B.Cu") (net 10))
 (segment (start 185.42 127) (end 185.415106 127) (width 0.8) (layer "F.Cu") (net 9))
 (segment (start 170.182439 111.767333) (end 170.182439 111.757561) (width 0.8) (layer "F.Cu") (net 9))
 (segment (start 185.415106 127) (end 170.182439 111.767333) (width 0.8) (layer "F.Cu") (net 9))
 (via (at 185.42 127) (size 1.8) (drill 0.8) (layers "F.Cu" "B.Cu") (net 9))
 (via (at 170.182439 111.757561) (size 1.8) (drill 0.8) (layers "F.Cu" "B.Cu") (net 9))
 (segment (start 170.182439 110.492439) (end 167.64 107.95) (width 0.8) (layer "B.Cu") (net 9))
 (segment (start 185.42 129.54) (end 185.42 127) (width 0.8) (layer "B.Cu") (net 9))
 (segment (start 170.182439 111.757561) (end 170.182439 110.492439) (width 0.8) (layer "B.Cu") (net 9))
 (segment (start 193.04 137.16) (end 185.42 129.54) (width 0.8) (layer "B.Cu") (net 9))
 (segment (start 186.425068 110.541009) (end 192.677217 110.541009) (width 0.8) (layer "F.Cu") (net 4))
 (segment (start 192.677217 110.541009) (end 192.751647 110.466579) (width 0.8) (layer "F.Cu") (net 4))
 (via (at 192.751647 110.466579) (size 1.8) (drill 0.8) (layers "F.Cu" "B.Cu") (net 4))
 (via (at 186.425068 110.541009) (size 1.8) (drill 0.8) (layers "F.Cu" "B.Cu") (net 4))
 (segment (start 192.751647 109.508353) (end 195.58 106.68) (width 0.8) (layer "B.Cu") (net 4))
 (segment (start 162.56 107.95) (end 164.259511 106.250489) (width 0.8) (layer "B.Cu") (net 4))
 (segment (start 182.134548 106.250489) (end 186.425068 110.541009) (width 0.8) (layer "B.Cu") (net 4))
 (segment (start 192.751647 110.466579) (end 192.751647 109.508353) (width 0.8) (layer "B.Cu") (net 4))
 (segment (start 164.259511 106.250489) (end 182.134548 106.250489) (width 0.8) (layer "B.Cu") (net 4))
 (segment (start 195.58 99.06) (end 195.58 129.54) (width 0.8) (layer "B.Cu") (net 4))
 (segment (start 192.428116 125.556167) (end 186.521061 125.556167) (width 0.8) (layer "F.Cu") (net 12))
 (segment (start 175.264894 114.3) (end 175.26 114.3) (width 0.8) (layer "F.Cu") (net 12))
 (segment (start 186.521061 125.556167) (end 175.264894 114.3) (width 0.8) (layer "F.Cu") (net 12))
 (segment (start 192.928096 126.056147) (end 192.428116 125.556167) (width 0.8) (layer "F.Cu") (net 12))
 (via (at 175.26 114.3) (size 1.8) (drill 0.8) (layers "F.Cu" "B.Cu") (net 12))
 (via (at 192.928096 126.056147) (size 1.8) (drill 0.8) (layers "F.Cu" "B.Cu") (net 12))
 (segment (start 192.928096 126.056147) (end 193.04 126.168051) (width 0.8) (layer "B.Cu") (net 12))
 (segment (start 175.26 114.3) (end 166.37 114.3) (width 0.8) (layer "B.Cu") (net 12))
 (segment (start 193.04 126.168051) (end 193.04 129.54) (width 0.8) (layer "B.Cu") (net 12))
 (segment (start 166.37 114.3) (end 160.02 107.95) (width 0.8) (layer "B.Cu") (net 12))
 (segment (start 191.290489 116.049511) (end 165.579511 116.049511) (width 0.8) (layer "B.Cu") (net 24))
 (segment (start 165.579511 116.049511) (end 157.48 107.95) (width 0.8) (layer "B.Cu") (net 24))
 (segment (start 193.04 114.3) (end 191.290489 116.049511) (width 0.8) (layer "B.Cu") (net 24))
 (segment (start 193.04 121.92) (end 188.469031 117.349031) (width 0.8) (layer "B.Cu") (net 5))
 (segment (start 188.469031 117.349031) (end 164.339031 117.349031) (width 0.8) (layer "B.Cu") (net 5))
 (segment (start 164.339031 117.349031) (end 154.94 107.95) (width 0.8) (layer "B.Cu") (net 5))
 (segment (start 193.04 106.68) (end 189.25952 102.89952) (width 0.8) (layer "B.Cu") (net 25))
 (segment (start 157.45048 102.89952) (end 152.4 107.95) (width 0.8) (layer "B.Cu") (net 25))
 (segment (start 189.25952 102.89952) (end 157.45048 102.89952) (width 0.8) (layer "B.Cu") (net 25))
 (segment (start 190.5 101.6) (end 154.94 101.6) (width 0.8) (layer "B.Cu") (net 26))
 (segment (start 193.04 99.06) (end 190.5 101.6) (width 0.8) (layer "B.Cu") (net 26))
 (segment (start 154.94 101.6) (end 149.86 106.68) (width 0.8) (layer "B.Cu") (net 26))
 (segment (start 149.86 106.68) (end 149.86 107.95) (width 0.8) (layer "B.Cu") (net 26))
 (segment (start 180.34 129.54) (end 167.39 129.54) (width 0.8) (layer "B.Cu") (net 11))
 (segment (start 167.39 129.54) (end 145.8 107.95) (width 0.8) (layer "B.Cu") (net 11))
 (segment (start 187.96 137.16) (end 180.34 129.54) (width 0.8) (layer "B.Cu") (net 11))
 (segment (start 197.485 83.82) (end 159.77 83.82) (width 0.8) (layer "B.Cu") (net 30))
 (segment (start 200.66 80.645) (end 197.485 83.82) (width 0.8) (layer "B.Cu") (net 30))
 (segment (start 159.77 83.82) (end 135.64 107.95) (width 0.8) (layer "B.Cu") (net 30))
 (segment (start 187.96 152.4) (end 147.32 111.76) (width 0.8) (layer "B.Cu") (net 35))
 (segment (start 126.75 111.76) (end 122.94 107.95) (width 0.8) (layer "B.Cu") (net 35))
 (segment (start 195.58 151.819022) (end 194.999022 152.4) (width 0.8) (layer "B.Cu") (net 35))
 (segment (start 194.999022 152.4) (end 187.96 152.4) (width 0.8) (layer "B.Cu") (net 35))
 (segment (start 147.32 111.76) (end 126.75 111.76) (width 0.8) (layer "B.Cu") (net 35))
 (segment (start 195.58 144.78) (end 195.58 151.819022) (width 0.8) (layer "B.Cu") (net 35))
 (segment (start 191.494843 71.12) (end 198.479843 78.105) (width 1.3) (layer "B.Cu") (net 36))
 (segment (start 200.694357 78.070643) (end 200.66 78.105) (width 1.3) (layer "B.Cu") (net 36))
 (segment (start 207.99113 78.070643) (end 200.694357 78.070643) (width 1.3) (layer "B.Cu") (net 36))
 (segment (start 190.5 71.12) (end 191.494843 71.12) (width 1.3) (layer "B.Cu") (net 36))
 (segment (start 198.479843 78.105) (end 200.66 78.105) (width 1.3) (layer "B.Cu") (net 36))
 (segment (start 193.04 143.577919) (end 198.12 138.497919) (width 1.3) (layer "B.Cu") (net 3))
 (segment (start 193.04 149.86) (end 193.04 144.78) (width 1.3) (layer "B.Cu") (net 3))
 (segment (start 198.12 138.497919) (end 198.12 137.16) (width 1.3) (layer "B.Cu") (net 3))
 (segment (start 193.04 144.78) (end 193.04 143.577919) (width 1.3) (layer "B.Cu") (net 3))
 (segment (start 200.66 91.44) (end 198.12 93.98) (width 0.8) (layer "B.Cu") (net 1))
 (segment (start 198.12 93.98) (end 198.12 99.06) (width 0.8) (layer "B.Cu") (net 1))
 (segment (start 198.12 114.3) (end 198.12 121.92) (width 0.8) (layer "B.Cu") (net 1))
 (segment (start 200.66 88.9) (end 200.66 91.44) (width 0.8) (layer "B.Cu") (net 1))
 (segment (start 198.12 99.06) (end 198.12 106.68) (width 0.8) (layer "B.Cu") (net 1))
 (segment (start 198.12 106.68) (end 198.12 114.3) (width 0.8) (layer "B.Cu") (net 1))
 (segment (start 198.12 121.92) (end 198.12 129.54) (width 0.8) (layer "B.Cu") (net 1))
 (segment (start 212.38252 65.501284) (end 205.836284 65.501284) (width 0.8) (layer "B.Cu") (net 7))
 (segment (start 205.836284 65.501284) (end 205.74 65.405) (width 0.8) (layer "B.Cu") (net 7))
 (segment (start 190.5 65.405) (end 198.12 65.405) (width 0.8) (layer "B.Cu") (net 7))
 (segment (start 205.74 65.405) (end 198.12 65.405) (width 0.8) (layer "B.Cu") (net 7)))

